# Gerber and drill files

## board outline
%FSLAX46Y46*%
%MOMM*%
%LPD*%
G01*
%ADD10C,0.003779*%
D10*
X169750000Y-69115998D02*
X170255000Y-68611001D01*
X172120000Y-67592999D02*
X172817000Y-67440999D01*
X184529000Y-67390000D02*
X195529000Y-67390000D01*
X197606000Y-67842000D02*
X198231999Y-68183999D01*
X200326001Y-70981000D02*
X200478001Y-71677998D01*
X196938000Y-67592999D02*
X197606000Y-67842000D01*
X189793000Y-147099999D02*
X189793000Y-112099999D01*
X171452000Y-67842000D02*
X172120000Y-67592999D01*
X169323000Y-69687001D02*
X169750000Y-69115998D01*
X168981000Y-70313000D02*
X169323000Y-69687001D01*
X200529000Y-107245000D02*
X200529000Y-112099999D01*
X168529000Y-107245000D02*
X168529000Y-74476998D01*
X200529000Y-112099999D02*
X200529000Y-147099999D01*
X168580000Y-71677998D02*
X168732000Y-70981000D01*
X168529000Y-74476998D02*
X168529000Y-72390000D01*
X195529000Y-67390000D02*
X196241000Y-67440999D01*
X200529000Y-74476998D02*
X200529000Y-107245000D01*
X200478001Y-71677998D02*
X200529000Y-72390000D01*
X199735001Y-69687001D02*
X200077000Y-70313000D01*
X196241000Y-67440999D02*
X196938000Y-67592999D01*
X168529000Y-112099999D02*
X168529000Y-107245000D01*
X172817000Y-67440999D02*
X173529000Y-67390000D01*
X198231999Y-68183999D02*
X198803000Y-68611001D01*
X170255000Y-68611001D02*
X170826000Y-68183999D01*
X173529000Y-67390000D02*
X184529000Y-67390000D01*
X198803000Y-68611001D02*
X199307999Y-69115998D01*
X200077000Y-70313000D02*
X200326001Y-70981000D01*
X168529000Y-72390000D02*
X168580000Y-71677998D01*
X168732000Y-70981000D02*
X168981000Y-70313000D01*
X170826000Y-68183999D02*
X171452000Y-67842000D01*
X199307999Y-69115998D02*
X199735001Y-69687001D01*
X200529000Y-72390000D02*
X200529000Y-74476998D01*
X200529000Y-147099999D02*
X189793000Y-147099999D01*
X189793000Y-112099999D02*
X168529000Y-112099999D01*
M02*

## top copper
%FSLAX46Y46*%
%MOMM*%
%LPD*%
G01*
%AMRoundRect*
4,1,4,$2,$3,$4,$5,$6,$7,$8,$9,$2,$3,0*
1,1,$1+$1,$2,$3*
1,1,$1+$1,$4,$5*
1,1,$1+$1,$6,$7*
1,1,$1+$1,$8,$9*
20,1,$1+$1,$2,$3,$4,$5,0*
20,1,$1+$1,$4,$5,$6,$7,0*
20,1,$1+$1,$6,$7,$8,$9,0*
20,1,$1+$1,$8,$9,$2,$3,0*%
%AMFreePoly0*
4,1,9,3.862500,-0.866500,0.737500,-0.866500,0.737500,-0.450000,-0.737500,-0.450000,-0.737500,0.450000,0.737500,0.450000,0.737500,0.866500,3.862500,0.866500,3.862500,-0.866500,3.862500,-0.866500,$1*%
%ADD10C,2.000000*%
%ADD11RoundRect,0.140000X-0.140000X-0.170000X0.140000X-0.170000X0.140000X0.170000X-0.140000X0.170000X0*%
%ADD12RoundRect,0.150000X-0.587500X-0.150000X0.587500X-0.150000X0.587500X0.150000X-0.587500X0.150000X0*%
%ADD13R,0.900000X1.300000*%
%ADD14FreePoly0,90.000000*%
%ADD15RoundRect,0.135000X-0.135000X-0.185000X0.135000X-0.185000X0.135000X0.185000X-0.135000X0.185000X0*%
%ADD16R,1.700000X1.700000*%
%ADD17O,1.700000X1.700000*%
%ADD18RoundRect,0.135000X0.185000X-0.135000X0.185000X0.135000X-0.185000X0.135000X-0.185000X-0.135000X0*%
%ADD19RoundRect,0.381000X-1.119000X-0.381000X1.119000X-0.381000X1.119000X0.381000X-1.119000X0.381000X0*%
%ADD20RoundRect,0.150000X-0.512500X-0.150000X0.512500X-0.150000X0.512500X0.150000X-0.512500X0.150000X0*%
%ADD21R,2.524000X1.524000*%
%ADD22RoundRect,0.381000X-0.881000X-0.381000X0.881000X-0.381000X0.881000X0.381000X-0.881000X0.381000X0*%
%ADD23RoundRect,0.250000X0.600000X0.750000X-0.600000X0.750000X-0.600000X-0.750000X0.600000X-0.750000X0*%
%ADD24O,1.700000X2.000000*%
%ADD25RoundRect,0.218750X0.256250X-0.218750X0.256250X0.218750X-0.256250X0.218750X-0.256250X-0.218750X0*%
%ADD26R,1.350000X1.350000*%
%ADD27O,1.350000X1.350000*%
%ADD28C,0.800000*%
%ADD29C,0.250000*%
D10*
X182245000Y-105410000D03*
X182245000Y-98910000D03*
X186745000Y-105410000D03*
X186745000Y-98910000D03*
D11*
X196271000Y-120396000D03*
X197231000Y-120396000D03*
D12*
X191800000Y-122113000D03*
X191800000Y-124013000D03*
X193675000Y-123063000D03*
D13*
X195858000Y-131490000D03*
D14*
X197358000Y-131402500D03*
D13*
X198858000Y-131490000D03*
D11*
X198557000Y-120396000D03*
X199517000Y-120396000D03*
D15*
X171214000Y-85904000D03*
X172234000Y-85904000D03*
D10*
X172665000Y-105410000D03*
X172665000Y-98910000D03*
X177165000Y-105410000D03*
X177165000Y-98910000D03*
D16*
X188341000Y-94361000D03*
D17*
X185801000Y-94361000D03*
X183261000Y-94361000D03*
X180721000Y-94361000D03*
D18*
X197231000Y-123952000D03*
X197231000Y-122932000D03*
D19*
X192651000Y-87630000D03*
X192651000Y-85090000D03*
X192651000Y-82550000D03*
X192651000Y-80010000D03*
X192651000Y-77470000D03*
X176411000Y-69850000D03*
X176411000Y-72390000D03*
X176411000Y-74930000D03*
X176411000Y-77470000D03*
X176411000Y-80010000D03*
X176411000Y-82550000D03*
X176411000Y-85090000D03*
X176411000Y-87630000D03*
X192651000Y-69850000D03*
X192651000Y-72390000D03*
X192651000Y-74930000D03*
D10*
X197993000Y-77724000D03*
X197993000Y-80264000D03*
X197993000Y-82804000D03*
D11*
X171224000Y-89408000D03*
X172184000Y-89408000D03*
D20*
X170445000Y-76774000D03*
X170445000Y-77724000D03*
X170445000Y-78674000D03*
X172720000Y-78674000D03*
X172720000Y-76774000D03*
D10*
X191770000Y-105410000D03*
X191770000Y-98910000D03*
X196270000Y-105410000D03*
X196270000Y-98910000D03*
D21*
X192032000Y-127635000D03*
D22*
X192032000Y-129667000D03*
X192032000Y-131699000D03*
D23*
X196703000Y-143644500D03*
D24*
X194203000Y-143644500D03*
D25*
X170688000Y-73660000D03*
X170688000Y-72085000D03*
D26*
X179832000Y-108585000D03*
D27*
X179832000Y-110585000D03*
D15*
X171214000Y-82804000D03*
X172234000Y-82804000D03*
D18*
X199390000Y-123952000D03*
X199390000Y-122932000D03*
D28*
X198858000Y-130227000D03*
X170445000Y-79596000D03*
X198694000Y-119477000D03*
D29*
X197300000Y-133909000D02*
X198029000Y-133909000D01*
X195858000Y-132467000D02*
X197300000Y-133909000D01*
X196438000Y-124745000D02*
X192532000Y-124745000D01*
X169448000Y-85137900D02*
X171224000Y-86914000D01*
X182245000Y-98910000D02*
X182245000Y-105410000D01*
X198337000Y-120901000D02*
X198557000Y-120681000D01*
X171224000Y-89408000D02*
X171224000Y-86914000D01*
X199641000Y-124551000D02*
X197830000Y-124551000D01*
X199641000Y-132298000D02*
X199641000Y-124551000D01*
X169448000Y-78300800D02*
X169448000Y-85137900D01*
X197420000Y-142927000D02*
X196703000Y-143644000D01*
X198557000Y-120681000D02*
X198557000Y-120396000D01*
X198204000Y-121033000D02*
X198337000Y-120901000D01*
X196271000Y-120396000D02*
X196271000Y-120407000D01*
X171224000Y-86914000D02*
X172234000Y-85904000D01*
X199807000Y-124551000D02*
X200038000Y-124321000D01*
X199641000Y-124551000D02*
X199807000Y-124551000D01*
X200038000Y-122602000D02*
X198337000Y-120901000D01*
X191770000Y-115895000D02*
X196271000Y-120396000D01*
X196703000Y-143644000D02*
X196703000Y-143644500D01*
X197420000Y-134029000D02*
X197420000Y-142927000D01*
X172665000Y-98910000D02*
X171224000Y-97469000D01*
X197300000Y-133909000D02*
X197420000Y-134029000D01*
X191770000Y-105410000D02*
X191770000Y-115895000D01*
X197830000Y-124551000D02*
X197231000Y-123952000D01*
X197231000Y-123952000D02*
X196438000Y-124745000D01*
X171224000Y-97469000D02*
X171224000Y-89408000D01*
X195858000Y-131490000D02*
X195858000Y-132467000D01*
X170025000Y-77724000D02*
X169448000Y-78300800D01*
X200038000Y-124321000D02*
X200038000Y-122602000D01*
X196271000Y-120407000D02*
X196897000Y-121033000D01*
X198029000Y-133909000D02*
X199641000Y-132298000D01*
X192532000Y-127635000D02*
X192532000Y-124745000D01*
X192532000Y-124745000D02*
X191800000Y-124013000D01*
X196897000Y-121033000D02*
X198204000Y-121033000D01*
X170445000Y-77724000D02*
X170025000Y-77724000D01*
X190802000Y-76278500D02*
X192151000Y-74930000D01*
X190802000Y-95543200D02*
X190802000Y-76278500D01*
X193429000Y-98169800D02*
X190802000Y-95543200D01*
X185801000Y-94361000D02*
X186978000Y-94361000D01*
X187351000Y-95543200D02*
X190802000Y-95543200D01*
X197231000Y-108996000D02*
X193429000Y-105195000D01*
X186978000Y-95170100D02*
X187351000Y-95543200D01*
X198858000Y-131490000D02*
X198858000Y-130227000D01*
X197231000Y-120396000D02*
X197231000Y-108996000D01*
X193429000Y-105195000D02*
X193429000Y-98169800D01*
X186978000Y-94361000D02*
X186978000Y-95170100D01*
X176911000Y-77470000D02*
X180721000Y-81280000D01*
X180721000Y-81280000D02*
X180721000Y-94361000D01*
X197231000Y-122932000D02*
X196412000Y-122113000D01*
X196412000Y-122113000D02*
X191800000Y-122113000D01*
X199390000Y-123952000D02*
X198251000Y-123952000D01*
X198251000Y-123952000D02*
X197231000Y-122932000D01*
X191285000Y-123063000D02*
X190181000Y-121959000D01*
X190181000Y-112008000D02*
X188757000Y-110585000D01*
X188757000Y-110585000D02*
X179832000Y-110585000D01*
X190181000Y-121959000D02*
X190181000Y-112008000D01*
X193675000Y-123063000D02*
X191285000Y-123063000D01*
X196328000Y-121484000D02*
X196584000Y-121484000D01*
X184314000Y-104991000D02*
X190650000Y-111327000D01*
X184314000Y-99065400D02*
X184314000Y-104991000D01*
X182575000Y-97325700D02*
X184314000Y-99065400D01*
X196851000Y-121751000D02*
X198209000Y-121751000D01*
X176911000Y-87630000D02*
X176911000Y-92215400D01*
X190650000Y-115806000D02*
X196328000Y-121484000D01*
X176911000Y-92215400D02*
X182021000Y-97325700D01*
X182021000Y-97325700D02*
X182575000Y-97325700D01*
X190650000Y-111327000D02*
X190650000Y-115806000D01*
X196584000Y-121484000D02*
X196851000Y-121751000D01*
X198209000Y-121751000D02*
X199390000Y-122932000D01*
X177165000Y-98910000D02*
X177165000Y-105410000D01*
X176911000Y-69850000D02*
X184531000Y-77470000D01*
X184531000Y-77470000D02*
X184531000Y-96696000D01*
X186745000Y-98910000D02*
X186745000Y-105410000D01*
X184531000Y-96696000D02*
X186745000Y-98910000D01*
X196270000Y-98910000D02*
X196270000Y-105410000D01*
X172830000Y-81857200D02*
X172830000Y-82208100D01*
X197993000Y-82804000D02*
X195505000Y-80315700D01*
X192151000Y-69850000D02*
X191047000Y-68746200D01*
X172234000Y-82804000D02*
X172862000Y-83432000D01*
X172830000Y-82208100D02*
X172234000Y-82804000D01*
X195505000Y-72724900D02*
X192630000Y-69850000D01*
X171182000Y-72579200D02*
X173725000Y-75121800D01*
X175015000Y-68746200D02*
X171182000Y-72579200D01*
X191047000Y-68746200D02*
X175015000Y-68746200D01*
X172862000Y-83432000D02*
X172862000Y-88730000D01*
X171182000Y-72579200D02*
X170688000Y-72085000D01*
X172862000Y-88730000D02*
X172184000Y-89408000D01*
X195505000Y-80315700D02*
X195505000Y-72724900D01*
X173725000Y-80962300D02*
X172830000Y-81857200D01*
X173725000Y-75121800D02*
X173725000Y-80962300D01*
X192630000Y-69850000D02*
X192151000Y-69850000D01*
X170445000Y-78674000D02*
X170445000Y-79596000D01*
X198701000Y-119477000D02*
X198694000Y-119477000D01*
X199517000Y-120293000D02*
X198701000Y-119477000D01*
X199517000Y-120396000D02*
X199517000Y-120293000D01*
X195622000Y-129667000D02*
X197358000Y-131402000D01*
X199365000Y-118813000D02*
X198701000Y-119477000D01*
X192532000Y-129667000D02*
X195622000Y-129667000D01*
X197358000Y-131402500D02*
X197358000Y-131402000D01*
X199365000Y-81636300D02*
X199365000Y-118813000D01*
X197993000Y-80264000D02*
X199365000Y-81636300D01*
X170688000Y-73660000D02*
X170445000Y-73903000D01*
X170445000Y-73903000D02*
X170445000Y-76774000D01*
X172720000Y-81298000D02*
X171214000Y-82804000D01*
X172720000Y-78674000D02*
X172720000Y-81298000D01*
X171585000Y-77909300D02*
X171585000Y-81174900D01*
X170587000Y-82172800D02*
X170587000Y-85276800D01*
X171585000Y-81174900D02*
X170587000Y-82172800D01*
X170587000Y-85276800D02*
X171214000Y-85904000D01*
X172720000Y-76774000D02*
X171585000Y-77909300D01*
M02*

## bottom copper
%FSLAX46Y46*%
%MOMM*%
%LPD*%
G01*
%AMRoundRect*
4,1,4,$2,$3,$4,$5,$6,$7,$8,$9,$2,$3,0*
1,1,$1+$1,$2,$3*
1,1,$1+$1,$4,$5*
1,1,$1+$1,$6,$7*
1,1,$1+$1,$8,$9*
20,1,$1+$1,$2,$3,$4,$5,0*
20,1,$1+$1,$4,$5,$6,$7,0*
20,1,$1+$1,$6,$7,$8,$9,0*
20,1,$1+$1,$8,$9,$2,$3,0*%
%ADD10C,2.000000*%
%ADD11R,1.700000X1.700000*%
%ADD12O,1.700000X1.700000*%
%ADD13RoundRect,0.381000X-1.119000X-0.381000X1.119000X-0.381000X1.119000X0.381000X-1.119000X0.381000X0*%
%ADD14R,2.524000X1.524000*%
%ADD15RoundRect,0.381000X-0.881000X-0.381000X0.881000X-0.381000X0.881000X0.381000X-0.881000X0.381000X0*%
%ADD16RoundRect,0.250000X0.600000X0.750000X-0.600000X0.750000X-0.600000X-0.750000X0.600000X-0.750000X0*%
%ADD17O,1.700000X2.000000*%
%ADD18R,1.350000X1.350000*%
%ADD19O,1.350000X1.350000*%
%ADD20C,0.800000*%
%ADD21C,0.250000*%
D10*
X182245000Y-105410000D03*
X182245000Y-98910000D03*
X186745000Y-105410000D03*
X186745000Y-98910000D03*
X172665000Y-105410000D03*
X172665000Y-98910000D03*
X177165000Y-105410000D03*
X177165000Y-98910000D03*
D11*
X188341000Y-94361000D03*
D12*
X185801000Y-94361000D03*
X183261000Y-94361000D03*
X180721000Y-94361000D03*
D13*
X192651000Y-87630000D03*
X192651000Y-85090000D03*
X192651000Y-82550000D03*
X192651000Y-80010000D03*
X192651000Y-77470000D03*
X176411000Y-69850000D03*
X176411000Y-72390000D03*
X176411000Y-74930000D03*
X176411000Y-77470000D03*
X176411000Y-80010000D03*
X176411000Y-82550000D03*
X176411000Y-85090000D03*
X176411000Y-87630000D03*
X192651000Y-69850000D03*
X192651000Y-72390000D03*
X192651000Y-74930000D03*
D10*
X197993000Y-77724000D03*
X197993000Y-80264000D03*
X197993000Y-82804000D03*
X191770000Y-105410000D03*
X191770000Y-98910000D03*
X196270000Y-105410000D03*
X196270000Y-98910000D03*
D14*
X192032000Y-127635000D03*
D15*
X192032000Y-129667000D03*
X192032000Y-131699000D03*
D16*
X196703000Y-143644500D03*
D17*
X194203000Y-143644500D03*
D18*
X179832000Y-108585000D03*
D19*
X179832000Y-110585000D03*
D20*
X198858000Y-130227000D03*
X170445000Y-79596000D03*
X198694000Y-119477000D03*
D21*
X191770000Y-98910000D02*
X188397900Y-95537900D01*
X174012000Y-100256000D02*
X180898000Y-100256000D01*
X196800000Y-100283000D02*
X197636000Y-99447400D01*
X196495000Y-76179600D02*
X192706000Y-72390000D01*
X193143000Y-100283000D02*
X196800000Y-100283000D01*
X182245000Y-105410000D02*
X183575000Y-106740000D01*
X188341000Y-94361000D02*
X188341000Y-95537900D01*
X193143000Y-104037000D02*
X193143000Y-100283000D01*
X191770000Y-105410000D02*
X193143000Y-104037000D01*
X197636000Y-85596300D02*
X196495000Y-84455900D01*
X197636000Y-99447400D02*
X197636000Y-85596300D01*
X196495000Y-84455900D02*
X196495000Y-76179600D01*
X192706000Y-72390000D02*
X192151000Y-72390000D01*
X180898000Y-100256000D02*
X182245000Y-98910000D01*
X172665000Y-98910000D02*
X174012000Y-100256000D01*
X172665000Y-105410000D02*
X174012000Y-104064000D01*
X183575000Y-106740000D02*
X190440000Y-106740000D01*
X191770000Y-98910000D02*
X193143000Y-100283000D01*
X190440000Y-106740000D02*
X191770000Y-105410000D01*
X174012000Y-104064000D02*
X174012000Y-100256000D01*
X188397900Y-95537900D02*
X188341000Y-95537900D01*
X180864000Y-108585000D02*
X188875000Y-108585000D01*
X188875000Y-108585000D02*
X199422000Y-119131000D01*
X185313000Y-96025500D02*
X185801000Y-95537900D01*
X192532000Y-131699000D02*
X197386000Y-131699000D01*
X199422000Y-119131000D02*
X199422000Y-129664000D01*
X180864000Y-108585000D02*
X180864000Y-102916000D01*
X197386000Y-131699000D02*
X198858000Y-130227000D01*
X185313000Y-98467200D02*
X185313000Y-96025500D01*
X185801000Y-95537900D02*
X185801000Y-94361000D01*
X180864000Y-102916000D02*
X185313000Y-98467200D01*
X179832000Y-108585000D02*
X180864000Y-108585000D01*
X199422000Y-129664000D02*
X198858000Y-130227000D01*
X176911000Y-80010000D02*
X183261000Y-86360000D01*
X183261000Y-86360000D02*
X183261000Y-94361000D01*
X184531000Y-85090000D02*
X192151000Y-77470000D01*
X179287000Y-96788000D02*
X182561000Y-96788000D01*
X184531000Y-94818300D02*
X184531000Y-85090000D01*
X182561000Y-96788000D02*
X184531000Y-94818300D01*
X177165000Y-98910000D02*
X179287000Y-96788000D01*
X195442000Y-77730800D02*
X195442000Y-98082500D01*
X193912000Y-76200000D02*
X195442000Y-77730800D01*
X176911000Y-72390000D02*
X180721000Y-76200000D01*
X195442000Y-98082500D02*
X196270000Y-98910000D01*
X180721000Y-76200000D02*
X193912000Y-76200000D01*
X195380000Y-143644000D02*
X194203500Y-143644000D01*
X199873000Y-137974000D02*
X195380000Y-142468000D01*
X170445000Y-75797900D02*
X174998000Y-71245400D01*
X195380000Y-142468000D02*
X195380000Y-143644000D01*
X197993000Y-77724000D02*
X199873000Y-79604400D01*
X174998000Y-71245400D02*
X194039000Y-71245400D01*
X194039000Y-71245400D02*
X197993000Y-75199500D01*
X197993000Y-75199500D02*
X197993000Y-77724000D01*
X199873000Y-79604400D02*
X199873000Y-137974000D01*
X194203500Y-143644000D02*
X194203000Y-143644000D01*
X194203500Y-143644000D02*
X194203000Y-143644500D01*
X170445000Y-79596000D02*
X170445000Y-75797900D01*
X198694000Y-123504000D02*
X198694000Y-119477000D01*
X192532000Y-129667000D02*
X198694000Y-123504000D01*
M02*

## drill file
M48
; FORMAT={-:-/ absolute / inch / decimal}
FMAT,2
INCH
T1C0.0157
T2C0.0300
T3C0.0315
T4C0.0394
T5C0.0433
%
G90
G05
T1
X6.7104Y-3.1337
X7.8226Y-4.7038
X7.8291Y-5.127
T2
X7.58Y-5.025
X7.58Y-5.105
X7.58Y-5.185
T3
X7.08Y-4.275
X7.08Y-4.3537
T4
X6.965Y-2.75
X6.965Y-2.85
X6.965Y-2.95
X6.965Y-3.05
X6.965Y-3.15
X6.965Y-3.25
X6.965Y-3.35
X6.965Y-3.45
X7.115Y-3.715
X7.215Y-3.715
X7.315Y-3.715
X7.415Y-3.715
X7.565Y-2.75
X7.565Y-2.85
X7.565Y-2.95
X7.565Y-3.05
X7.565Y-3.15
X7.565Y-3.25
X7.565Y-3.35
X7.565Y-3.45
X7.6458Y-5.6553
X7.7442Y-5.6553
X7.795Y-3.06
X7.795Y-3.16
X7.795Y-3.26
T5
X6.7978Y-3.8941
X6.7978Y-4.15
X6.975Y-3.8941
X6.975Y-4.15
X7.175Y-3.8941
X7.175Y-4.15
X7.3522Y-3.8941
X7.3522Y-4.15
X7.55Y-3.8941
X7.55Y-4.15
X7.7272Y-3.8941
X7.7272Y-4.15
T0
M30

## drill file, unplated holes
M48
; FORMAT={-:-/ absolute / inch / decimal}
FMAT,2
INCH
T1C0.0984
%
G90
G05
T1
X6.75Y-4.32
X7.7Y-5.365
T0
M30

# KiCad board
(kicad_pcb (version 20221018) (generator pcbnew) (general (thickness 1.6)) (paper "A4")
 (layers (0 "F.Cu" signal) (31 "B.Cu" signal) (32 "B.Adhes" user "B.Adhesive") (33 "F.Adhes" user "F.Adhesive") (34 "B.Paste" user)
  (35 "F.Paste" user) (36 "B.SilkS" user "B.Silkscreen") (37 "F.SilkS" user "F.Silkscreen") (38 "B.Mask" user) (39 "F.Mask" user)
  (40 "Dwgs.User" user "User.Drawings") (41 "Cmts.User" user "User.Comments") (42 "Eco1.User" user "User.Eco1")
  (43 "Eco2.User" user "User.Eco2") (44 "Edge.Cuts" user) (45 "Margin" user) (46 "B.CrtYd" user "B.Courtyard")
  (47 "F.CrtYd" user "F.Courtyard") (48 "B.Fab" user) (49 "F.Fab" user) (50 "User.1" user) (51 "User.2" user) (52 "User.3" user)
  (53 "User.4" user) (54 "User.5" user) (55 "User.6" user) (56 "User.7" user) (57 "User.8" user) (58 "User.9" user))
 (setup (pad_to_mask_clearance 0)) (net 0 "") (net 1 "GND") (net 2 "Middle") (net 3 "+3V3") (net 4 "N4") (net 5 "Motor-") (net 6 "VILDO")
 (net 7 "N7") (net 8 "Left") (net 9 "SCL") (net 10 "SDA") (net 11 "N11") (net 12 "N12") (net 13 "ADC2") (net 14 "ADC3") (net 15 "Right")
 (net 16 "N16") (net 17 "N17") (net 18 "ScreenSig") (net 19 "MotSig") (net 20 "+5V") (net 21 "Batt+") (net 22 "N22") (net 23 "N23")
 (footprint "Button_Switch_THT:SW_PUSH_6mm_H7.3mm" (layer "F.Cu") (at 182.245 105.41 90)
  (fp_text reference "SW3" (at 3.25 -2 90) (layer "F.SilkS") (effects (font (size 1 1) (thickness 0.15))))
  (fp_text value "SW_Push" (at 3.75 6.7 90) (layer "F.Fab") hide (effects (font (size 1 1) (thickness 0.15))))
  (pad "1" thru_hole circle (at 0 0 180) (size 2 2) (drill 1.1) (layers "*.Cu" "*.Mask") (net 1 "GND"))
  (pad "1" thru_hole circle (at 6.5 0 180) (size 2 2) (drill 1.1) (layers "*.Cu" "*.Mask") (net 1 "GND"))
  (pad "2" thru_hole circle (at 0 4.5 180) (size 2 2) (drill 1.1) (layers "*.Cu" "*.Mask") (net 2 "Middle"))
  (pad "2" thru_hole circle (at 6.5 4.5 180) (size 2 2) (drill 1.1) (layers "*.Cu" "*.Mask") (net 2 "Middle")))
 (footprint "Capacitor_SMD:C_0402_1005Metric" (layer "F.Cu") (at 196.751 120.396)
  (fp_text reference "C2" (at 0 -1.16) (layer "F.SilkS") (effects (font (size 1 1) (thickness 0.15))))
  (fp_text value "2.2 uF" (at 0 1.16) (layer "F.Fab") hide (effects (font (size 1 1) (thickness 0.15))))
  (pad "1" smd roundrect (at -0.48 0) (size 0.56 0.62) (layers "F.Cu" "F.Paste" "F.Mask") (roundrect_rratio 0.25) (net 1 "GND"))
  (pad "2" smd roundrect (at 0.48 0) (size 0.56 0.62) (layers "F.Cu" "F.Paste" "F.Mask") (roundrect_rratio 0.25) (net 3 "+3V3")))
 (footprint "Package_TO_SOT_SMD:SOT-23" (layer "F.Cu") (at 192.7375 123.063)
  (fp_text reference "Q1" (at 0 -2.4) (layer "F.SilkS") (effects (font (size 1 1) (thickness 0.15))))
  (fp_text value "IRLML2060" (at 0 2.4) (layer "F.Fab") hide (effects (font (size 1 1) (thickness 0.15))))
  (pad "1" smd roundrect (at -0.9375 -0.95) (size 1.475 0.6) (layers "F.Cu" "F.Paste" "F.Mask") (roundrect_rratio 0.25) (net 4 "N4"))
  (pad "2" smd roundrect (at -0.9375 0.95) (size 1.475 0.6) (layers "F.Cu" "F.Paste" "F.Mask") (roundrect_rratio 0.25) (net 1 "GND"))
  (pad "3" smd roundrect (at 0.9375 0) (size 1.475 0.6) (layers "F.Cu" "F.Paste" "F.Mask") (roundrect_rratio 0.25) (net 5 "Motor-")))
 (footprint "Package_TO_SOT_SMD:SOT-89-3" (layer "F.Cu") (at 197.358 129.54 90)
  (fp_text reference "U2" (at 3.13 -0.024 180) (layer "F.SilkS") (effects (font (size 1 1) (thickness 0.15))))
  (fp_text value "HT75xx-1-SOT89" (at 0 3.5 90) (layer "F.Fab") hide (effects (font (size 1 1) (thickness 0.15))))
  (pad "1" smd rect (at -1.95 -1.5 90) (size 1.3 0.9) (layers "F.Cu" "F.Paste" "F.Mask") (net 1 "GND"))
  (pad "2" smd custom (at -1.8625 0 90) (size 1.475 0.9) (layers "F.Cu" "F.Paste" "F.Mask") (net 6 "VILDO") (zone_connect 2)
   (thermal_bridge_angle 45) (options (clearance outline) (anchor rect)) (primitives))
  (pad "3" smd rect (at -1.95 1.5 90) (size 1.3 0.9) (layers "F.Cu" "F.Paste" "F.Mask") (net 3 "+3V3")))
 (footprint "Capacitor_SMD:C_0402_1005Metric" (layer "F.Cu") (at 199.037 120.396)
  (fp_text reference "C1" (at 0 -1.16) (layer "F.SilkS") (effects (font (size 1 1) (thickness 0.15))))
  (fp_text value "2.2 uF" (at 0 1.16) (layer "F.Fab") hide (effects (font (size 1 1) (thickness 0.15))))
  (pad "1" smd roundrect (at -0.48 0) (size 0.56 0.62) (layers "F.Cu" "F.Paste" "F.Mask") (roundrect_rratio 0.25) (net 1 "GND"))
  (pad "2" smd roundrect (at 0.48 0) (size 0.56 0.62) (layers "F.Cu" "F.Paste" "F.Mask") (roundrect_rratio 0.25) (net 6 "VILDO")))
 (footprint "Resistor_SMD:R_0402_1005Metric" (layer "F.Cu") (at 171.724 85.904)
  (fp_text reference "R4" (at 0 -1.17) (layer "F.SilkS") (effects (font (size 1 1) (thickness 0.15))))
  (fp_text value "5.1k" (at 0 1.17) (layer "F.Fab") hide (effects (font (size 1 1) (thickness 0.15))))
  (pad "1" smd roundrect (at -0.51 0) (size 0.54 0.64) (layers "F.Cu" "F.Paste" "F.Mask") (roundrect_rratio 0.25) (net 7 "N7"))
  (pad "2" smd roundrect (at 0.51 0) (size 0.54 0.64) (layers "F.Cu" "F.Paste" "F.Mask") (roundrect_rratio 0.25) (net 1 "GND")))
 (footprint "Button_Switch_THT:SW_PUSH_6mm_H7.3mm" (layer "F.Cu") (at 172.665 105.41 90)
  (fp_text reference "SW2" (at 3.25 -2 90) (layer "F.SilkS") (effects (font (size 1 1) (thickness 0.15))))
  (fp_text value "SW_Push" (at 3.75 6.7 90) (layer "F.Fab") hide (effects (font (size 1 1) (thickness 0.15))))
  (pad "1" thru_hole circle (at 0 0 180) (size 2 2) (drill 1.1) (layers "*.Cu" "*.Mask") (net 1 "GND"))
  (pad "1" thru_hole circle (at 6.5 0 180) (size 2 2) (drill 1.1) (layers "*.Cu" "*.Mask") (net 1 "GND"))
  (pad "2" thru_hole circle (at 0 4.5 180) (size 2 2) (drill 1.1) (layers "*.Cu" "*.Mask") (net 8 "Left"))
  (pad "2" thru_hole circle (at 6.5 4.5 180) (size 2 2) (drill 1.1) (layers "*.Cu" "*.Mask") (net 8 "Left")))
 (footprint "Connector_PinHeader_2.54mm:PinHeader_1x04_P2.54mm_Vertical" (layer "F.Cu") (at 188.341 94.361 -90)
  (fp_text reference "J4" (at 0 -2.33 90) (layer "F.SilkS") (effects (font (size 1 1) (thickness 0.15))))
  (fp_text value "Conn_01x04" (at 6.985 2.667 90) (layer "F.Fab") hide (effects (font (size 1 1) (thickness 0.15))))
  (pad "1" thru_hole rect (at 0 0 270) (size 1.7 1.7) (drill 1) (layers "*.Cu" "*.Mask") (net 1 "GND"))
  (pad "2" thru_hole oval (at 0 2.54 270) (size 1.7 1.7) (drill 1) (layers "*.Cu" "*.Mask") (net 3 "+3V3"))
  (pad "3" thru_hole oval (at 0 5.08 270) (size 1.7 1.7) (drill 1) (layers "*.Cu" "*.Mask") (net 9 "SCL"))
  (pad "4" thru_hole oval (at 0 7.62 270) (size 1.7 1.7) (drill 1) (layers "*.Cu" "*.Mask") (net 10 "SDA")))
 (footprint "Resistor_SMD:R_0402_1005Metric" (layer "F.Cu") (at 197.231 123.442 90)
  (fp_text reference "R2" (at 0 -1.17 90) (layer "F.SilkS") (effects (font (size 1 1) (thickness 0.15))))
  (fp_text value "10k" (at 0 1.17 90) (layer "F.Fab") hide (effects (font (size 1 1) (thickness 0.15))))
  (pad "1" smd roundrect (at -0.51 0 90) (size 0.54 0.64) (layers "F.Cu" "F.Paste" "F.Mask") (roundrect_rratio 0.25) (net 1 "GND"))
  (pad "2" smd roundrect (at 0.51 0 90) (size 0.54 0.64) (layers "F.Cu" "F.Paste" "F.Mask") (roundrect_rratio 0.25) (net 4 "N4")))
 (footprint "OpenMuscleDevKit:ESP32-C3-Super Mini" (layer "F.Cu") (at 184.531 69.85)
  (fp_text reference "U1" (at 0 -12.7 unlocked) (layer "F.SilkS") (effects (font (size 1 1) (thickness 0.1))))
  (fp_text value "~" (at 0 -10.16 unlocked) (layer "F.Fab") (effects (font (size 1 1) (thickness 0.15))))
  (pad "0" thru_hole roundrect (at 7.62 17.78) (size 3 1.524) (drill 1 (offset 0.5 0)) (layers "*.Cu" "*.Mask") (roundrect_rratio 0.25)
   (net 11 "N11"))
  (pad "1" thru_hole roundrect (at 7.62 15.24) (size 3 1.524) (drill 1 (offset 0.5 0)) (layers "*.Cu" "*.Mask") (roundrect_rratio 0.25)
   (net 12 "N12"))
  (pad "2" thru_hole roundrect (at 7.62 12.7) (size 3 1.524) (drill 1 (offset 0.5 0)) (layers "*.Cu" "*.Mask") (roundrect_rratio 0.25)
   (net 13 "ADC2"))
  (pad "3" thru_hole roundrect (at 7.62 10.16) (size 3 1.524) (drill 1 (offset 0.5 0)) (layers "*.Cu" "*.Mask") (roundrect_rratio 0.25)
   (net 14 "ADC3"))
  (pad "4" thru_hole roundrect (at 7.62 7.62) (size 3 1.524) (drill 1 (offset 0.5 0)) (layers "*.Cu" "*.Mask") (roundrect_rratio 0.25)
   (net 8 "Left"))
  (pad "5" thru_hole roundrect (at -7.62 0) (size 3 1.524) (drill 1 (offset -0.5 0)) (layers "*.Cu" "*.Mask") (roundrect_rratio 0.25)
   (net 2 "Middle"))
  (pad "6" thru_hole roundrect (at -7.62 2.54) (size 3 1.524) (drill 1 (offset -0.5 0)) (layers "*.Cu" "*.Mask") (roundrect_rratio 0.25)
   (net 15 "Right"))
  (pad "7" thru_hole roundrect (at -7.62 5.08) (size 3 1.524) (drill 1 (offset -0.5 0)) (layers "*.Cu" "*.Mask") (roundrect_rratio 0.25)
   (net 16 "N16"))
  (pad "8" thru_hole roundrect (at -7.62 7.62) (size 3 1.524) (drill 1 (offset -0.5 0)) (layers "*.Cu" "*.Mask") (roundrect_rratio 0.25)
   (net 10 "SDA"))
  (pad "9" thru_hole roundrect (at -7.62 10.16) (size 3 1.524) (drill 1 (offset -0.5 0)) (layers "*.Cu" "*.Mask") (roundrect_rratio 0.25)
   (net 9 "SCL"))
  (pad "10" thru_hole roundrect (at -7.62 12.7) (size 3 1.524) (drill 1 (offset -0.5 0)) (layers "*.Cu" "*.Mask") (roundrect_rratio 0.25)
   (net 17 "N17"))
  (pad "20" thru_hole roundrect (at -7.62 15.24) (size 3 1.524) (drill 1 (offset -0.5 0)) (layers "*.Cu" "*.Mask") (roundrect_rratio 0.25)
   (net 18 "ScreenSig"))
  (pad "21" thru_hole roundrect (at -7.62 17.78) (size 3 1.524) (drill 1 (offset -0.5 0)) (layers "*.Cu" "*.Mask") (roundrect_rratio 0.25)
   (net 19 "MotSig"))
  (pad "100" thru_hole roundrect (at 7.62 0) (size 3 1.524) (drill 1 (offset 0.5 0)) (layers "*.Cu" "*.Mask") (roundrect_rratio 0.25)
   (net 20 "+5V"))
  (pad "101" thru_hole roundrect (at 7.62 2.54) (size 3 1.524) (drill 1 (offset 0.5 0)) (layers "*.Cu" "*.Mask") (roundrect_rratio 0.25)
   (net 1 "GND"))
  (pad "102" thru_hole roundrect (at 7.62 5.08) (size 3 1.524) (drill 1 (offset 0.5 0)) (layers "*.Cu" "*.Mask") (roundrect_rratio 0.25)
   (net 3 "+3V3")))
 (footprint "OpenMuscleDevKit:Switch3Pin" (layer "F.Cu") (at 197.993 81.534)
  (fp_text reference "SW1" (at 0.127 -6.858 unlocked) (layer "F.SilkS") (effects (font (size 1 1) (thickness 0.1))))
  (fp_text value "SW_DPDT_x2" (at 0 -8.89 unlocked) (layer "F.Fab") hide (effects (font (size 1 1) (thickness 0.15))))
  (pad "1" thru_hole circle (at 0 -3.81) (size 2 2) (drill 1) (layers "*.Cu" "*.Mask") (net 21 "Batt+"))
  (pad "2" thru_hole circle (at 0 -1.27) (size 2 2) (drill 1) (layers "*.Cu" "*.Mask") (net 6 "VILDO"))
  (pad "3" thru_hole circle (at 0 1.27) (size 2 2) (drill 1) (layers "*.Cu" "*.Mask") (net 20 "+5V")))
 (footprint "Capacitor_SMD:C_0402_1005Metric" (layer "F.Cu") (at 171.704 89.408)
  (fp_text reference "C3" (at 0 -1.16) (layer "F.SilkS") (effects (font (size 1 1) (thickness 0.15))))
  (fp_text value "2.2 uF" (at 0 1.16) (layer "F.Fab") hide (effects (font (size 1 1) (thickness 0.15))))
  (pad "1" smd roundrect (at -0.48 0) (size 0.56 0.62) (layers "F.Cu" "F.Paste" "F.Mask") (roundrect_rratio 0.25) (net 1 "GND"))
  (pad "2" smd roundrect (at 0.48 0) (size 0.56 0.62) (layers "F.Cu" "F.Paste" "F.Mask") (roundrect_rratio 0.25) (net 20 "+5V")))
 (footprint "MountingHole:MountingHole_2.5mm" (layer "F.Cu") (at 195.58 136.271)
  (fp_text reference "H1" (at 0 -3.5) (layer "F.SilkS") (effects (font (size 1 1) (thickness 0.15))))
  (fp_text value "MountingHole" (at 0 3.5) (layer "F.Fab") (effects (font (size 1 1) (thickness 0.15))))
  (pad "" np_thru_hole circle (at 0 0) (size 2.5 2.5) (drill 2.5) (layers "*.Cu" "*.Mask")))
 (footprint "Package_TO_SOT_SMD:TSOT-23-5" (layer "F.Cu") (at 171.5825 77.724)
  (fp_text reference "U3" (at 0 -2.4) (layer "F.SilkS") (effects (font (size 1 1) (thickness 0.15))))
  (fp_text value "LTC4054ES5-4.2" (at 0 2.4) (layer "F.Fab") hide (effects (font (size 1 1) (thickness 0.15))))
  (pad "1" smd roundrect (at -1.1375 -0.95) (size 1.325 0.6) (layers "F.Cu" "F.Paste" "F.Mask") (roundrect_rratio 0.25) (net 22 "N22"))
  (pad "2" smd roundrect (at -1.1375 0) (size 1.325 0.6) (layers "F.Cu" "F.Paste" "F.Mask") (roundrect_rratio 0.25) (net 1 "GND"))
  (pad "3" smd roundrect (at -1.1375 0.95) (size 1.325 0.6) (layers "F.Cu" "F.Paste" "F.Mask") (roundrect_rratio 0.25) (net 21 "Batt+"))
  (pad "4" smd roundrect (at 1.1375 0.95) (size 1.325 0.6) (layers "F.Cu" "F.Paste" "F.Mask") (roundrect_rratio 0.25) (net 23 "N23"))
  (pad "5" smd roundrect (at 1.1375 -0.95) (size 1.325 0.6) (layers "F.Cu" "F.Paste" "F.Mask") (roundrect_rratio 0.25) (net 7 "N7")))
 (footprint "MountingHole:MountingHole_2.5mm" (layer "F.Cu") (at 171.45 109.728)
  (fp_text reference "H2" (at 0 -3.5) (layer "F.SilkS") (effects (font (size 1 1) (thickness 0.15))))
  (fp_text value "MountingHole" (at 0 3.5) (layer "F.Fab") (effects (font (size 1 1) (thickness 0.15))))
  (pad "" np_thru_hole circle (at 0 0) (size 2.5 2.5) (drill 2.5) (layers "*.Cu" "*.Mask")))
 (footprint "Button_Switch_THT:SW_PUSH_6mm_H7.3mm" (layer "F.Cu") (at 191.77 105.41 90)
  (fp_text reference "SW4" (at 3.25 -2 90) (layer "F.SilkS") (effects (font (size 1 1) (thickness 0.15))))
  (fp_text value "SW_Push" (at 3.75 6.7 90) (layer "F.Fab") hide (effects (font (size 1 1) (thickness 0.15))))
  (pad "1" thru_hole circle (at 0 0 180) (size 2 2) (drill 1.1) (layers "*.Cu" "*.Mask") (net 1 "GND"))
  (pad "1" thru_hole circle (at 6.5 0 180) (size 2 2) (drill 1.1) (layers "*.Cu" "*.Mask") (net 1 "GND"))
  (pad "2" thru_hole circle (at 0 4.5 180) (size 2 2) (drill 1.1) (layers "*.Cu" "*.Mask") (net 15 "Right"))
  (pad "2" thru_hole circle (at 6.5 4.5 180) (size 2 2) (drill 1.1) (layers "*.Cu" "*.Mask") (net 15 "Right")))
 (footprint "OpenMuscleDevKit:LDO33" (layer "F.Cu") (at 194.096 130.175 -90)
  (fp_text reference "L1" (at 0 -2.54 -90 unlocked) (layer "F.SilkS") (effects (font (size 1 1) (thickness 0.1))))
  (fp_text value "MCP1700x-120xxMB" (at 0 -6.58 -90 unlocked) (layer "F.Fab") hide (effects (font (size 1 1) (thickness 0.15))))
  (pad "1" thru_hole rect (at -2.54 1.564) (size 2.524 1.524) (drill 0.762 (offset -0.5 0)) (layers "*.Cu" "*.Mask") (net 1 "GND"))
  (pad "2" thru_hole roundrect (at -0.508 1.564) (size 2.524 1.524) (drill 0.762 (offset -0.5 0)) (layers "*.Cu" "*.Mask")
   (roundrect_rratio 0.25) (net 6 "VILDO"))
  (pad "3" thru_hole roundrect (at 1.524 1.564) (size 2.524 1.524) (drill 0.762 (offset -0.5 0)) (layers "*.Cu" "*.Mask")
   (roundrect_rratio 0.25) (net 3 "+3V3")))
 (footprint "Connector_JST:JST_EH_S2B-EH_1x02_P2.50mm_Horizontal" (layer "F.Cu") (at 196.703 143.6445 180)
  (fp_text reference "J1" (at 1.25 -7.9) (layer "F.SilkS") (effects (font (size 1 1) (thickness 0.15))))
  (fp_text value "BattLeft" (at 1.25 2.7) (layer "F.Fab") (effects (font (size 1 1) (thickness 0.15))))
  (pad "1" thru_hole roundrect (at 0 0 180) (size 1.7 2) (drill 1) (layers "*.Cu" "*.Mask") (roundrect_rratio 0.1470588235) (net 1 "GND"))
  (pad "2" thru_hole oval (at 2.5 0 180) (size 1.7 2) (drill 1) (layers "*.Cu" "*.Mask") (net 21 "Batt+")))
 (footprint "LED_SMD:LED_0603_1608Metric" (layer "F.Cu") (at 170.688 72.8725 90)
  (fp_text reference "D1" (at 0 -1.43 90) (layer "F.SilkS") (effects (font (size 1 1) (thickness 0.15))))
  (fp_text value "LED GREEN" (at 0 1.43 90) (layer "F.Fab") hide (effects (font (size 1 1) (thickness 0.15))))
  (pad "1" smd roundrect (at -0.7875 0 90) (size 0.875 0.95) (layers "F.Cu" "F.Paste" "F.Mask") (roundrect_rratio 0.25) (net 22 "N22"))
  (pad "2" smd roundrect (at 0.7875 0 90) (size 0.875 0.95) (layers "F.Cu" "F.Paste" "F.Mask") (roundrect_rratio 0.25) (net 20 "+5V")))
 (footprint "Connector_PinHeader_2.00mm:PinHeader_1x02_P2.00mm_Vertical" (layer "F.Cu") (at 179.832 108.585)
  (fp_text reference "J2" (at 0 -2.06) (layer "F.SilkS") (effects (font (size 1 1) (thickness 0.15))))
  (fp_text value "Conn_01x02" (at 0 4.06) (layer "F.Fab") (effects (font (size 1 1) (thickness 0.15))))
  (pad "1" thru_hole rect (at 0 0) (size 1.35 1.35) (drill 0.8) (layers "*.Cu" "*.Mask") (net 3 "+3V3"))
  (pad "2" thru_hole oval (at 0 2) (size 1.35 1.35) (drill 0.8) (layers "*.Cu" "*.Mask") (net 5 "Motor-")))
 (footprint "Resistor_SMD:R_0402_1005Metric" (layer "F.Cu") (at 171.724 82.804)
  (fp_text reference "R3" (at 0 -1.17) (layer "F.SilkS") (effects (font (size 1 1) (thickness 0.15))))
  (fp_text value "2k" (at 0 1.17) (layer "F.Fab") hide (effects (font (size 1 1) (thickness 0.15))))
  (pad "1" smd roundrect (at -0.51 0) (size 0.54 0.64) (layers "F.Cu" "F.Paste" "F.Mask") (roundrect_rratio 0.25) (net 23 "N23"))
  (pad "2" smd roundrect (at 0.51 0) (size 0.54 0.64) (layers "F.Cu" "F.Paste" "F.Mask") (roundrect_rratio 0.25) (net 20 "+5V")))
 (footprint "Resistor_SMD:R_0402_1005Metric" (layer "F.Cu") (at 199.39 123.442 90)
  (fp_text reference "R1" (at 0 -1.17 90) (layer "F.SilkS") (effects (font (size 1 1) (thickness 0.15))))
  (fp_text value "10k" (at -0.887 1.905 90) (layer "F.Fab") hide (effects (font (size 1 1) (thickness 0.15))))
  (pad "1" smd roundrect (at -0.51 0 90) (size 0.54 0.64) (layers "F.Cu" "F.Paste" "F.Mask") (roundrect_rratio 0.25) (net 4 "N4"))
  (pad "2" smd roundrect (at 0.51 0 90) (size 0.54 0.64) (layers "F.Cu" "F.Paste" "F.Mask") (roundrect_rratio 0.25) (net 19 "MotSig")))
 (gr_line (start 169.75 69.115998) (end 170.255 68.611001) (stroke (width 0.003779) (type solid)) (layer "Edge.Cuts"))
 (gr_line (start 172.12 67.592999) (end 172.817 67.440999) (stroke (width 0.003779) (type solid)) (layer "Edge.Cuts"))
 (gr_line (start 184.529 67.39) (end 195.529 67.39) (stroke (width 0.003779) (type solid)) (layer "Edge.Cuts"))
 (gr_line (start 197.606 67.842) (end 198.231999 68.183999) (stroke (width 0.003779) (type solid)) (layer "Edge.Cuts"))
 (gr_line (start 200.326001 70.981) (end 200.478001 71.677998) (stroke (width 0.003779) (type solid)) (layer "Edge.Cuts"))
 (gr_line (start 196.938 67.592999) (end 197.606 67.842) (stroke (width 0.003779) (type solid)) (layer "Edge.Cuts"))
 (gr_line (start 189.793 147.099999) (end 189.793 112.099999) (stroke (width 0.003779) (type solid)) (layer "Edge.Cuts"))
 (gr_line (start 171.452 67.842) (end 172.12 67.592999) (stroke (width 0.003779) (type solid)) (layer "Edge.Cuts"))
 (gr_line (start 169.323 69.687001) (end 169.75 69.115998) (stroke (width 0.003779) (type solid)) (layer "Edge.Cuts"))
 (gr_line (start 168.981 70.313) (end 169.323 69.687001) (stroke (width 0.003779) (type solid)) (layer "Edge.Cuts"))
 (gr_line (start 200.529 107.245) (end 200.529 112.099999) (stroke (width 0.003779) (type solid)) (layer "Edge.Cuts"))
 (gr_line (start 168.529 107.245) (end 168.529 74.476998) (stroke (width 0.003779) (type solid)) (layer "Edge.Cuts"))
 (gr_line (start 200.529 112.099999) (end 200.529 147.099999) (stroke (width 0.003779) (type solid)) (layer "Edge.Cuts"))
 (gr_line (start 168.58 71.677998) (end 168.732 70.981) (stroke (width 0.003779) (type solid)) (layer "Edge.Cuts"))
 (gr_line (start 168.529 74.476998) (end 168.529 72.39) (stroke (width 0.003779) (type solid)) (layer "Edge.Cuts"))
 (gr_line (start 195.529 67.39) (end 196.241 67.440999) (stroke (width 0.003779) (type solid)) (layer "Edge.Cuts"))
 (gr_line (start 200.529 74.476998) (end 200.529 107.245) (stroke (width 0.003779) (type solid)) (layer "Edge.Cuts"))
 (gr_line (start 200.478001 71.677998) (end 200.529 72.39) (stroke (width 0.003779) (type solid)) (layer "Edge.Cuts"))
 (gr_line (start 199.735001 69.687001) (end 200.077 70.313) (stroke (width 0.003779) (type solid)) (layer "Edge.Cuts"))
 (gr_line (start 196.241 67.440999) (end 196.938 67.592999) (stroke (width 0.003779) (type solid)) (layer "Edge.Cuts"))
 (gr_line (start 168.529 112.099999) (end 168.529 107.245) (stroke (width 0.003779) (type solid)) (layer "Edge.Cuts"))
 (gr_line (start 172.817 67.440999) (end 173.529 67.39) (stroke (width 0.003779) (type solid)) (layer "Edge.Cuts"))
 (gr_line (start 198.231999 68.183999) (end 198.803 68.611001) (stroke (width 0.003779) (type solid)) (layer "Edge.Cuts"))
 (gr_line (start 170.255 68.611001) (end 170.826 68.183999) (stroke (width 0.003779) (type solid)) (layer "Edge.Cuts"))
 (gr_line (start 173.529 67.39) (end 184.529 67.39) (stroke (width 0.003779) (type solid)) (layer "Edge.Cuts"))
 (gr_line (start 198.803 68.611001) (end 199.307999 69.115998) (stroke (width 0.003779) (type solid)) (layer "Edge.Cuts"))
 (gr_line (start 200.077 70.313) (end 200.326001 70.981) (stroke (width 0.003779) (type solid)) (layer "Edge.Cuts"))
 (gr_line (start 168.529 72.39) (end 168.58 71.677998) (stroke (width 0.003779) (type solid)) (layer "Edge.Cuts"))
 (gr_line (start 168.732 70.981) (end 168.981 70.313) (stroke (width 0.003779) (type solid)) (layer "Edge.Cuts"))
 (gr_line (start 170.826 68.183999) (end 171.452 67.842) (stroke (width 0.003779) (type solid)) (layer "Edge.Cuts"))
 (gr_line (start 199.307999 69.115998) (end 199.735001 69.687001) (stroke (width 0.003779) (type solid)) (layer "Edge.Cuts"))
 (gr_line (start 200.529 72.39) (end 200.529 74.476998) (stroke (width 0.003779) (type solid)) (layer "Edge.Cuts"))
 (gr_line (start 200.529 147.099999) (end 189.793 147.099999) (stroke (width 0.003779) (type solid)) (layer "Edge.Cuts"))
 (gr_line (start 189.793 112.099999) (end 168.529 112.099999) (stroke (width 0.003779) (type solid)) (layer "Edge.Cuts"))
 (segment (start 197.3 133.909) (end 198.029 133.909) (width 0.25) (layer "F.Cu") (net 1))
 (segment (start 195.858 132.467) (end 197.3 133.909) (width 0.25) (layer "F.Cu") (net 1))
 (segment (start 196.438 124.745) (end 192.532 124.745) (width 0.25) (layer "F.Cu") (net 1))
 (segment (start 169.448 85.1379) (end 171.224 86.914) (width 0.25) (layer "F.Cu") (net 1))
 (segment (start 182.245 98.91) (end 182.245 105.41) (width 0.25) (layer "F.Cu") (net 1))
 (segment (start 198.337 120.901) (end 198.557 120.681) (width 0.25) (layer "F.Cu") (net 1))
 (segment (start 171.224 89.408) (end 171.224 86.914) (width 0.25) (layer "F.Cu") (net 1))
 (segment (start 199.641 124.551) (end 197.83 124.551) (width 0.25) (layer "F.Cu") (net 1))
 (segment (start 199.641 132.298) (end 199.641 124.551) (width 0.25) (layer "F.Cu") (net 1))
 (segment (start 169.448 78.3008) (end 169.448 85.1379) (width 0.25) (layer "F.Cu") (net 1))
 (segment (start 197.42 142.927) (end 196.703 143.644) (width 0.25) (layer "F.Cu") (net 1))
 (segment (start 198.557 120.681) (end 198.557 120.396) (width 0.25) (layer "F.Cu") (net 1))
 (segment (start 198.204 121.033) (end 198.337 120.901) (width 0.25) (layer "F.Cu") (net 1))
 (segment (start 196.271 120.396) (end 196.271 120.407) (width 0.25) (layer "F.Cu") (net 1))
 (segment (start 171.224 86.914) (end 172.234 85.904) (width 0.25) (layer "F.Cu") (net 1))
 (segment (start 199.807 124.551) (end 200.038 124.321) (width 0.25) (layer "F.Cu") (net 1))
 (segment (start 199.641 124.551) (end 199.807 124.551) (width 0.25) (layer "F.Cu") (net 1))
 (segment (start 200.038 122.602) (end 198.337 120.901) (width 0.25) (layer "F.Cu") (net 1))
 (segment (start 191.77 115.895) (end 196.271 120.396) (width 0.25) (layer "F.Cu") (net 1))
 (segment (start 196.703 143.644) (end 196.703 143.6445) (width 0.25) (layer "F.Cu") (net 1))
 (segment (start 197.42 134.029) (end 197.42 142.927) (width 0.25) (layer "F.Cu") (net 1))
 (segment (start 172.665 98.91) (end 171.224 97.469) (width 0.25) (layer "F.Cu") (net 1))
 (segment (start 197.3 133.909) (end 197.42 134.029) (width 0.25) (layer "F.Cu") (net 1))
 (segment (start 191.77 105.41) (end 191.77 115.895) (width 0.25) (layer "F.Cu") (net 1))
 (segment (start 197.83 124.551) (end 197.231 123.952) (width 0.25) (layer "F.Cu") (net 1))
 (segment (start 197.231 123.952) (end 196.438 124.745) (width 0.25) (layer "F.Cu") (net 1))
 (segment (start 171.224 97.469) (end 171.224 89.408) (width 0.25) (layer "F.Cu") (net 1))
 (segment (start 195.858 131.49) (end 195.858 132.467) (width 0.25) (layer "F.Cu") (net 1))
 (segment (start 170.025 77.724) (end 169.448 78.3008) (width 0.25) (layer "F.Cu") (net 1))
 (segment (start 200.038 124.321) (end 200.038 122.602) (width 0.25) (layer "F.Cu") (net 1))
 (segment (start 196.271 120.407) (end 196.897 121.033) (width 0.25) (layer "F.Cu") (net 1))
 (segment (start 198.029 133.909) (end 199.641 132.298) (width 0.25) (layer "F.Cu") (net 1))
 (segment (start 192.532 127.635) (end 192.532 124.745) (width 0.25) (layer "F.Cu") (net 1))
 (segment (start 192.532 124.745) (end 191.8 124.013) (width 0.25) (layer "F.Cu") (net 1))
 (segment (start 196.897 121.033) (end 198.204 121.033) (width 0.25) (layer "F.Cu") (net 1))
 (segment (start 170.445 77.724) (end 170.025 77.724) (width 0.25) (layer "F.Cu") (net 1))
 (segment (start 191.77 98.91) (end 188.3979 95.5379) (width 0.25) (layer "B.Cu") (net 1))
 (segment (start 174.012 100.256) (end 180.898 100.256) (width 0.25) (layer "B.Cu") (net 1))
 (segment (start 196.8 100.283) (end 197.636 99.4474) (width 0.25) (layer "B.Cu") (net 1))
 (segment (start 196.495 76.1796) (end 192.706 72.39) (width 0.25) (layer "B.Cu") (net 1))
 (segment (start 193.143 100.283) (end 196.8 100.283) (width 0.25) (layer "B.Cu") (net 1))
 (segment (start 182.245 105.41) (end 183.575 106.74) (width 0.25) (layer "B.Cu") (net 1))
 (segment (start 188.341 94.361) (end 188.341 95.5379) (width 0.25) (layer "B.Cu") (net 1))
 (segment (start 193.143 104.037) (end 193.143 100.283) (width 0.25) (layer "B.Cu") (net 1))
 (segment (start 191.77 105.41) (end 193.143 104.037) (width 0.25) (layer "B.Cu") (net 1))
 (segment (start 197.636 85.5963) (end 196.495 84.4559) (width 0.25) (layer "B.Cu") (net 1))
 (segment (start 197.636 99.4474) (end 197.636 85.5963) (width 0.25) (layer "B.Cu") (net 1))
 (segment (start 196.495 84.4559) (end 196.495 76.1796) (width 0.25) (layer "B.Cu") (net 1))
 (segment (start 192.706 72.39) (end 192.151 72.39) (width 0.25) (layer "B.Cu") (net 1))
 (segment (start 180.898 100.256) (end 182.245 98.91) (width 0.25) (layer "B.Cu") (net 1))
 (segment (start 172.665 98.91) (end 174.012 100.256) (width 0.25) (layer "B.Cu") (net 1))
 (segment (start 172.665 105.41) (end 174.012 104.064) (width 0.25) (layer "B.Cu") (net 1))
 (segment (start 183.575 106.74) (end 190.44 106.74) (width 0.25) (layer "B.Cu") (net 1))
 (segment (start 191.77 98.91) (end 193.143 100.283) (width 0.25) (layer "B.Cu") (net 1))
 (segment (start 190.44 106.74) (end 191.77 105.41) (width 0.25) (layer "B.Cu") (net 1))
 (segment (start 174.012 104.064) (end 174.012 100.256) (width 0.25) (layer "B.Cu") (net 1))
 (segment (start 188.3979 95.5379) (end 188.341 95.5379) (width 0.25) (layer "B.Cu") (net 1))
 (segment (start 190.802 76.2785) (end 192.151 74.93) (width 0.25) (layer "F.Cu") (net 3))
 (segment (start 190.802 95.5432) (end 190.802 76.2785) (width 0.25) (layer "F.Cu") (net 3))
 (segment (start 193.429 98.1698) (end 190.802 95.5432) (width 0.25) (layer "F.Cu") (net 3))
 (segment (start 185.801 94.361) (end 186.978 94.361) (width 0.25) (layer "F.Cu") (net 3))
 (segment (start 187.351 95.5432) (end 190.802 95.5432) (width 0.25) (layer "F.Cu") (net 3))
 (segment (start 197.231 108.996) (end 193.429 105.195) (width 0.25) (layer "F.Cu") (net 3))
 (segment (start 186.978 95.1701) (end 187.351 95.5432) (width 0.25) (layer "F.Cu") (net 3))
 (segment (start 198.858 131.49) (end 198.858 130.227) (width 0.25) (layer "F.Cu") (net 3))
 (segment (start 197.231 120.396) (end 197.231 108.996) (width 0.25) (layer "F.Cu") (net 3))
 (segment (start 193.429 105.195) (end 193.429 98.1698) (width 0.25) (layer "F.Cu") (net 3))
 (segment (start 186.978 94.361) (end 186.978 95.1701) (width 0.25) (layer "F.Cu") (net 3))
 (via (at 198.858 130.227) (size 0.8) (drill 0.4) (layers "F.Cu" "B.Cu") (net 3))
 (segment (start 180.864 108.585) (end 188.875 108.585) (width 0.25) (layer "B.Cu") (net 3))
 (segment (start 188.875 108.585) (end 199.422 119.131) (width 0.25) (layer "B.Cu") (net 3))
 (segment (start 185.313 96.0255) (end 185.801 95.5379) (width 0.25) (layer "B.Cu") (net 3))
 (segment (start 192.532 131.699) (end 197.386 131.699) (width 0.25) (layer "B.Cu") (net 3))
 (segment (start 199.422 119.131) (end 199.422 129.664) (width 0.25) (layer "B.Cu") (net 3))
 (segment (start 180.864 108.585) (end 180.864 102.916) (width 0.25) (layer "B.Cu") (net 3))
 (segment (start 197.386 131.699) (end 198.858 130.227) (width 0.25) (layer "B.Cu") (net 3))
 (segment (start 185.313 98.4672) (end 185.313 96.0255) (width 0.25) (layer "B.Cu") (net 3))
 (segment (start 185.801 95.5379) (end 185.801 94.361) (width 0.25) (layer "B.Cu") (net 3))
 (segment (start 180.864 102.916) (end 185.313 98.4672) (width 0.25) (layer "B.Cu") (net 3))
 (segment (start 179.832 108.585) (end 180.864 108.585) (width 0.25) (layer "B.Cu") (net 3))
 (segment (start 199.422 129.664) (end 198.858 130.227) (width 0.25) (layer "B.Cu") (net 3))
 (segment (start 176.911 80.01) (end 183.261 86.36) (width 0.25) (layer "B.Cu") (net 9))
 (segment (start 183.261 86.36) (end 183.261 94.361) (width 0.25) (layer "B.Cu") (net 9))
 (segment (start 176.911 77.47) (end 180.721 81.28) (width 0.25) (layer "F.Cu") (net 10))
 (segment (start 180.721 81.28) (end 180.721 94.361) (width 0.25) (layer "F.Cu") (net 10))
 (segment (start 197.231 122.932) (end 196.412 122.113) (width 0.25) (layer "F.Cu") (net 4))
 (segment (start 196.412 122.113) (end 191.8 122.113) (width 0.25) (layer "F.Cu") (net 4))
 (segment (start 199.39 123.952) (end 198.251 123.952) (width 0.25) (layer "F.Cu") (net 4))
 (segment (start 198.251 123.952) (end 197.231 122.932) (width 0.25) (layer "F.Cu") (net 4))
 (segment (start 191.285 123.063) (end 190.181 121.959) (width 0.25) (layer "F.Cu") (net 5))
 (segment (start 190.181 112.008) (end 188.757 110.585) (width 0.25) (layer "F.Cu") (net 5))
 (segment (start 188.757 110.585) (end 179.832 110.585) (width 0.25) (layer "F.Cu") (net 5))
 (segment (start 190.181 121.959) (end 190.181 112.008) (width 0.25) (layer "F.Cu") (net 5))
 (segment (start 193.675 123.063) (end 191.285 123.063) (width 0.25) (layer "F.Cu") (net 5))
 (segment (start 196.328 121.484) (end 196.584 121.484) (width 0.25) (layer "F.Cu") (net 19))
 (segment (start 184.314 104.991) (end 190.65 111.327) (width 0.25) (layer "F.Cu") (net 19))
 (segment (start 184.314 99.0654) (end 184.314 104.991) (width 0.25) (layer "F.Cu") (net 19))
 (segment (start 182.575 97.3257) (end 184.314 99.0654) (width 0.25) (layer "F.Cu") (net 19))
 (segment (start 196.851 121.751) (end 198.209 121.751) (width 0.25) (layer "F.Cu") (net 19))
 (segment (start 176.911 87.63) (end 176.911 92.2154) (width 0.25) (layer "F.Cu") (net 19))
 (segment (start 190.65 115.806) (end 196.328 121.484) (width 0.25) (layer "F.Cu") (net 19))
 (segment (start 176.911 92.2154) (end 182.021 97.3257) (width 0.25) (layer "F.Cu") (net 19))
 (segment (start 182.021 97.3257) (end 182.575 97.3257) (width 0.25) (layer "F.Cu") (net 19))
 (segment (start 190.65 111.327) (end 190.65 115.806) (width 0.25) (layer "F.Cu") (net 19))
 (segment (start 196.584 121.484) (end 196.851 121.751) (width 0.25) (layer "F.Cu") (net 19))
 (segment (start 198.209 121.751) (end 199.39 122.932) (width 0.25) (layer "F.Cu") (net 19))
 (segment (start 177.165 98.91) (end 177.165 105.41) (width 0.25) (layer "F.Cu") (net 8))
 (segment (start 184.531 85.09) (end 192.151 77.47) (width 0.25) (layer "B.Cu") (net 8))
 (segment (start 179.287 96.788) (end 182.561 96.788) (width 0.25) (layer "B.Cu") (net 8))
 (segment (start 184.531 94.8183) (end 184.531 85.09) (width 0.25) (layer "B.Cu") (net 8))
 (segment (start 182.561 96.788) (end 184.531 94.8183) (width 0.25) (layer "B.Cu") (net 8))
 (segment (start 177.165 98.91) (end 179.287 96.788) (width 0.25) (layer "B.Cu") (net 8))
 (segment (start 176.911 69.85) (end 184.531 77.47) (width 0.25) (layer "F.Cu") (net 2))
 (segment (start 184.531 77.47) (end 184.531 96.696) (width 0.25) (layer "F.Cu") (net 2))
 (segment (start 186.745 98.91) (end 186.745 105.41) (width 0.25) (layer "F.Cu") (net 2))
 (segment (start 184.531 96.696) (end 186.745 98.91) (width 0.25) (layer "F.Cu") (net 2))
 (segment (start 196.27 98.91) (end 196.27 105.41) (width 0.25) (layer "F.Cu") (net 15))
 (segment (start 195.442 77.7308) (end 195.442 98.0825) (width 0.25) (layer "B.Cu") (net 15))
 (segment (start 193.912 76.2) (end 195.442 77.7308) (width 0.25) (layer "B.Cu") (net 15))
 (segment (start 176.911 72.39) (end 180.721 76.2) (width 0.25) (layer "B.Cu") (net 15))
 (segment (start 195.442 98.0825) (end 196.27 98.91) (width 0.25) (layer "B.Cu") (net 15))
 (segment (start 180.721 76.2) (end 193.912 76.2) (width 0.25) (layer "B.Cu") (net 15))
 (segment (start 172.83 81.8572) (end 172.83 82.2081) (width 0.25) (layer "F.Cu") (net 20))
 (segment (start 197.993 82.804) (end 195.505 80.3157) (width 0.25) (layer "F.Cu") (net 20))
 (segment (start 192.151 69.85) (end 191.047 68.7462) (width 0.25) (layer "F.Cu") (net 20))
 (segment (start 172.234 82.804) (end 172.862 83.432) (width 0.25) (layer "F.Cu") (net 20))
 (segment (start 172.83 82.2081) (end 172.234 82.804) (width 0.25) (layer "F.Cu") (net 20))
 (segment (start 195.505 72.7249) (end 192.63 69.85) (width 0.25) (layer "F.Cu") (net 20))
 (segment (start 171.182 72.5792) (end 173.725 75.1218) (width 0.25) (layer "F.Cu") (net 20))
 (segment (start 175.015 68.7462) (end 171.182 72.5792) (width 0.25) (layer "F.Cu") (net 20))
 (segment (start 191.047 68.7462) (end 175.015 68.7462) (width 0.25) (layer "F.Cu") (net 20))
 (segment (start 172.862 83.432) (end 172.862 88.73) (width 0.25) (layer "F.Cu") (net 20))
 (segment (start 171.182 72.5792) (end 170.688 72.085) (width 0.25) (layer "F.Cu") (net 20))
 (segment (start 172.862 88.73) (end 172.184 89.408) (width 0.25) (layer "F.Cu") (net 20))
 (segment (start 195.505 80.3157) (end 195.505 72.7249) (width 0.25) (layer "F.Cu") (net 20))
 (segment (start 173.725 80.9623) (end 172.83 81.8572) (width 0.25) (layer "F.Cu") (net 20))
 (segment (start 173.725 75.1218) (end 173.725 80.9623) (width 0.25) (layer "F.Cu") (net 20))
 (segment (start 192.63 69.85) (end 192.151 69.85) (width 0.25) (layer "F.Cu") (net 20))
 (segment (start 170.445 78.674) (end 170.445 79.596) (width 0.25) (layer "F.Cu") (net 21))
 (via (at 170.445 79.596) (size 0.8) (drill 0.4) (layers "F.Cu" "B.Cu") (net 21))
 (segment (start 195.38 143.644) (end 194.2035 143.644) (width 0.25) (layer "B.Cu") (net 21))
 (segment (start 199.873 137.974) (end 195.38 142.468) (width 0.25) (layer "B.Cu") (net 21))
 (segment (start 170.445 75.7979) (end 174.998 71.2454) (width 0.25) (layer "B.Cu") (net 21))
 (segment (start 195.38 142.468) (end 195.38 143.644) (width 0.25) (layer "B.Cu") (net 21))
 (segment (start 197.993 77.724) (end 199.873 79.6044) (width 0.25) (layer "B.Cu") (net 21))
 (segment (start 174.998 71.2454) (end 194.039 71.2454) (width 0.25) (layer "B.Cu") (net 21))
 (segment (start 194.039 71.2454) (end 197.993 75.1995) (width 0.25) (layer "B.Cu") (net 21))
 (segment (start 197.993 75.1995) (end 197.993 77.724) (width 0.25) (layer "B.Cu") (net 21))
 (segment (start 199.873 79.6044) (end 199.873 137.974) (width 0.25) (layer "B.Cu") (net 21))
 (segment (start 194.2035 143.644) (end 194.203 143.644) (width 0.25) (layer "B.Cu") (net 21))
 (segment (start 194.2035 143.644) (end 194.203 143.6445) (width 0.25) (layer "B.Cu") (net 21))
 (segment (start 170.445 79.596) (end 170.445 75.7979) (width 0.25) (layer "B.Cu") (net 21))
 (segment (start 198.701 119.477) (end 198.694 119.477) (width 0.25) (layer "F.Cu") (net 6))
 (segment (start 199.517 120.293) (end 198.701 119.477) (width 0.25) (layer "F.Cu") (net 6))
 (segment (start 199.517 120.396) (end 199.517 120.293) (width 0.25) (layer "F.Cu") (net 6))
 (segment (start 195.622 129.667) (end 197.358 131.402) (width 0.25) (layer "F.Cu") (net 6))
 (segment (start 199.365 118.813) (end 198.701 119.477) (width 0.25) (layer "F.Cu") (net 6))
 (segment (start 192.532 129.667) (end 195.622 129.667) (width 0.25) (layer "F.Cu") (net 6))
 (segment (start 197.358 131.4025) (end 197.358 131.402) (width 0.25) (layer "F.Cu") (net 6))
 (segment (start 199.365 81.6363) (end 199.365 118.813) (width 0.25) (layer "F.Cu") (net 6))
 (segment (start 197.993 80.264) (end 199.365 81.6363) (width 0.25) (layer "F.Cu") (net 6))
 (via (at 198.694 119.477) (size 0.8) (drill 0.4) (layers "F.Cu" "B.Cu") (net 6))
 (segment (start 198.694 123.504) (end 198.694 119.477) (width 0.25) (layer "B.Cu") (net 6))
 (segment (start 192.532 129.667) (end 198.694 123.504) (width 0.25) (layer "B.Cu") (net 6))
 (segment (start 170.688 73.66) (end 170.445 73.903) (width 0.25) (layer "F.Cu") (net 22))
 (segment (start 170.445 73.903) (end 170.445 76.774) (width 0.25) (layer "F.Cu") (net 22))
 (segment (start 172.72 81.298) (end 171.214 82.804) (width 0.25) (layer "F.Cu") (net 23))
 (segment (start 172.72 78.674) (end 172.72 81.298) (width 0.25) (layer "F.Cu") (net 23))
 (segment (start 171.585 77.9093) (end 171.585 81.1749) (width 0.25) (layer "F.Cu") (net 7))
 (segment (start 170.587 82.1728) (end 170.587 85.2768) (width 0.25) (layer "F.Cu") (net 7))
 (segment (start 171.585 81.1749) (end 170.587 82.1728) (width 0.25) (layer "F.Cu") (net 7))
 (segment (start 170.587 85.2768) (end 171.214 85.904) (width 0.25) (layer "F.Cu") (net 7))
 (segment (start 172.72 76.774) (end 171.585 77.9093) (width 0.25) (layer "F.Cu") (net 7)))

